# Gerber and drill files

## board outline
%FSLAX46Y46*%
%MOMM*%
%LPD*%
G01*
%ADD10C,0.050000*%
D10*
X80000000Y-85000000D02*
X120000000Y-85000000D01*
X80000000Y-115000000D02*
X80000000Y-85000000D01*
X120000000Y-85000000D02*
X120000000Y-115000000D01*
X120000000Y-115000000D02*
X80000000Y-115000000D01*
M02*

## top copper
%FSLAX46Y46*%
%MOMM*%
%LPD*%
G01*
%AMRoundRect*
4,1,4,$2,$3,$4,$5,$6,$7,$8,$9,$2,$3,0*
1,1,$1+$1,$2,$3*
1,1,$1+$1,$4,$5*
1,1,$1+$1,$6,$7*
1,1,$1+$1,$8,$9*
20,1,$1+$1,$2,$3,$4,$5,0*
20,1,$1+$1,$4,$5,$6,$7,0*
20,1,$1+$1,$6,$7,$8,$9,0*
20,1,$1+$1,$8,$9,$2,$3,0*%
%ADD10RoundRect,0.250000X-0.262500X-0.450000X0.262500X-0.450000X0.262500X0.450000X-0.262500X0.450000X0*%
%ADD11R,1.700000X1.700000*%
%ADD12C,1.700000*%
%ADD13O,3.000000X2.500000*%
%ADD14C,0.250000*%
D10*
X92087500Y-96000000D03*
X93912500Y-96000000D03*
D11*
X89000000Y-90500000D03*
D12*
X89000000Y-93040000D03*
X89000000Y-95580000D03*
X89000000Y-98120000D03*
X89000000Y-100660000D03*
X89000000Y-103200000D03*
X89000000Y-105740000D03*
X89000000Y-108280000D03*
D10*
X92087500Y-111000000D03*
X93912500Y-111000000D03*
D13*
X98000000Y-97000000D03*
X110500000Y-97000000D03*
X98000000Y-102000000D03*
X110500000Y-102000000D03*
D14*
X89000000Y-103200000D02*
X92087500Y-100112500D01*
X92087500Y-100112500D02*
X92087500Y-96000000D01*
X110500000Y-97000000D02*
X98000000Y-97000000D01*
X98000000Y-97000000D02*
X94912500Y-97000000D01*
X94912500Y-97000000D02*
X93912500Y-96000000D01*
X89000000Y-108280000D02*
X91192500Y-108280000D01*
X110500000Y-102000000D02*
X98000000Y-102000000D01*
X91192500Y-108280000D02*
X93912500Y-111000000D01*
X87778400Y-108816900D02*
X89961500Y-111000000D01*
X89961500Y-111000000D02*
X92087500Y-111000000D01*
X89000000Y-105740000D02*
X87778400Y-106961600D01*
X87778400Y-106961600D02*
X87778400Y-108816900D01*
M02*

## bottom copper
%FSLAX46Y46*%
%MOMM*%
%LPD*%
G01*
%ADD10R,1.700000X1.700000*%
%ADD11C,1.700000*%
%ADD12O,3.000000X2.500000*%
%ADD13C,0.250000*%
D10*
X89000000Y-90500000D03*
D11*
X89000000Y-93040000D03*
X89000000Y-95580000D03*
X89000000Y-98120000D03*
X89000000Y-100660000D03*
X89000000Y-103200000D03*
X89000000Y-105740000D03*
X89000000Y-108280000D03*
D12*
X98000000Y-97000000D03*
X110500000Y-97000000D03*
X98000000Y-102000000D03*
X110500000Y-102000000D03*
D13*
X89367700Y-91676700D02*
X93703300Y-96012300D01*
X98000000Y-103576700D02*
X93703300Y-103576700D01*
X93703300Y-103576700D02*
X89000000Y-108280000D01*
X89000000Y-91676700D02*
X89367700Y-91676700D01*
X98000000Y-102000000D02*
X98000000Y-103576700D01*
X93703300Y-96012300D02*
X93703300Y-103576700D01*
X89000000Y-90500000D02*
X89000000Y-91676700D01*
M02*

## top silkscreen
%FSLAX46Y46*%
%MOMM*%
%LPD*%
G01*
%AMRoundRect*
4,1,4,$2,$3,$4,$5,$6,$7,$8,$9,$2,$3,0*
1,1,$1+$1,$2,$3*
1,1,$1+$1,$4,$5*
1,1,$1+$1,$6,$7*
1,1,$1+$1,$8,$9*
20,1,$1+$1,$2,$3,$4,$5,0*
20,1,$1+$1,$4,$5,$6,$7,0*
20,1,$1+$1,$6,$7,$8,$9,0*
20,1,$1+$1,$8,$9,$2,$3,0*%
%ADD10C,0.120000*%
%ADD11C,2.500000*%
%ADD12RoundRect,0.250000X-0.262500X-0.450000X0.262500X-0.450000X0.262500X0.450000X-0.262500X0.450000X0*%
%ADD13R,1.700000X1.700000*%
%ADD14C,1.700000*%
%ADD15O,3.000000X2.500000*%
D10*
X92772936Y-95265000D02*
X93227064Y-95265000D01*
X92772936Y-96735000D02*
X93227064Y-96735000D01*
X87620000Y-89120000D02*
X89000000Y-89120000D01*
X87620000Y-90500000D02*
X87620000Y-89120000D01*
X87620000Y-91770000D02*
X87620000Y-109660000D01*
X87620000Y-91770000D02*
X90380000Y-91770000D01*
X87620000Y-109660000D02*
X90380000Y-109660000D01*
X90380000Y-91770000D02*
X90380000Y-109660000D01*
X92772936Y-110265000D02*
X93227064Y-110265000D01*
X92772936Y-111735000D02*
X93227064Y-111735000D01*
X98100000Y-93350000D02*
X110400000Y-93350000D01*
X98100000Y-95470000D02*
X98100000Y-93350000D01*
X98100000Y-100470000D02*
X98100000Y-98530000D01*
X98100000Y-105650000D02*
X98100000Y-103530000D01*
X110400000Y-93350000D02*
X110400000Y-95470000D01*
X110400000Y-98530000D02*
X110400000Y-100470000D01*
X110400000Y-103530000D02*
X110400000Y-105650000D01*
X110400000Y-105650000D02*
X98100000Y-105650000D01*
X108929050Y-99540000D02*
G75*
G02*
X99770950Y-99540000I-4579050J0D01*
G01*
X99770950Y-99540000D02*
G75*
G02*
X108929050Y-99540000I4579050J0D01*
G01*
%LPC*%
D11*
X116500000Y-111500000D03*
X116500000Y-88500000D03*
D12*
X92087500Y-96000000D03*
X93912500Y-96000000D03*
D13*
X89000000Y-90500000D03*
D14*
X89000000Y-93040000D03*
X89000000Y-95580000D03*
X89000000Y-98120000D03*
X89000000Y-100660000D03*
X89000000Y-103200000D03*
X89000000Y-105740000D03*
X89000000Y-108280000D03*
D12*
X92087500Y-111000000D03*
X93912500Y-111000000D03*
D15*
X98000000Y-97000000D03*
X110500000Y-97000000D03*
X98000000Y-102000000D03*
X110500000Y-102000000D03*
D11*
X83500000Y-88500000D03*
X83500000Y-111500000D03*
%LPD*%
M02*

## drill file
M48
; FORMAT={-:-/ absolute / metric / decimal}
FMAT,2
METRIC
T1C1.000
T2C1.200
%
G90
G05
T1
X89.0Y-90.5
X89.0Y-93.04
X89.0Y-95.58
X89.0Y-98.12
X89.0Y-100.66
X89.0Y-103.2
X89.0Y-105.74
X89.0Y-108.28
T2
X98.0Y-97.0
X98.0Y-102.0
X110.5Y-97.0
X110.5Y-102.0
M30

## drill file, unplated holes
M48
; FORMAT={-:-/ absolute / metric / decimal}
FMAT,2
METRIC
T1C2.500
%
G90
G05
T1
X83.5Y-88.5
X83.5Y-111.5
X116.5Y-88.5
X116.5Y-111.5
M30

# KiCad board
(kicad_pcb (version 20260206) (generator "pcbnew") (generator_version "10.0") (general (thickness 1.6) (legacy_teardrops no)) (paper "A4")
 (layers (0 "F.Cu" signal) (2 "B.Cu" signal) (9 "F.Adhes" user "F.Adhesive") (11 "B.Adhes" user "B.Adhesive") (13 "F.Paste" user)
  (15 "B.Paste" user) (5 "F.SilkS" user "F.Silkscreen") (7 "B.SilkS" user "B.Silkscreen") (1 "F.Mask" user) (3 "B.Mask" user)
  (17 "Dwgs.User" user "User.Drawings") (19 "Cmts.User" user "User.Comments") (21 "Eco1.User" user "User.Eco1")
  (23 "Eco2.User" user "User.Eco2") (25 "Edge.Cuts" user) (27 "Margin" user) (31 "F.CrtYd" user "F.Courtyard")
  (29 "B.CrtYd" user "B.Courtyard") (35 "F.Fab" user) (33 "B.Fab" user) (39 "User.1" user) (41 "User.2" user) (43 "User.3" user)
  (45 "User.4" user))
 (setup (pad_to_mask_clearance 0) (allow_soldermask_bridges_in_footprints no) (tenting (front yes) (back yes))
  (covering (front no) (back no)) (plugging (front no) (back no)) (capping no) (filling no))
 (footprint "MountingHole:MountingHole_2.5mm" (layer "F.Cu") (at 116.5 111.5)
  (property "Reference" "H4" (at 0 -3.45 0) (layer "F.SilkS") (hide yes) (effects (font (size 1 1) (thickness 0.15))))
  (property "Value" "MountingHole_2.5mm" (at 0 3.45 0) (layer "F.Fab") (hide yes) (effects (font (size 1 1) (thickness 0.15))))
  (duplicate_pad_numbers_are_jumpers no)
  (pad "" np_thru_hole circle (at 0 0) (size 2.5 2.5) (drill 2.5) (layers "*.Cu" "*.Mask")))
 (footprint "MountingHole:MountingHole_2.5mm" (layer "F.Cu") (at 116.5 88.5)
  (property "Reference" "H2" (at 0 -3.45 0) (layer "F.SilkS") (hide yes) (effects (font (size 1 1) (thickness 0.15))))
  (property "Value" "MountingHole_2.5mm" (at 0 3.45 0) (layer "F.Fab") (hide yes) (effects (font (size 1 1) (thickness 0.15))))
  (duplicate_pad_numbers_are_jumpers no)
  (pad "" np_thru_hole circle (at 0 0) (size 2.5 2.5) (drill 2.5) (layers "*.Cu" "*.Mask")))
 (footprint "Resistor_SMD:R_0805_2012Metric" (layer "F.Cu") (at 93 96)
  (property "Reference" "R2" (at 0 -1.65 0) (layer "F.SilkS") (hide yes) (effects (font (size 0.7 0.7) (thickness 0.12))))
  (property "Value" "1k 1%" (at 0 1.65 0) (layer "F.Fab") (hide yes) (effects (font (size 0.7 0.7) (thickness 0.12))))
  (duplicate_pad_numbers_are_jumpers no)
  (fp_line (start -0.227064 -0.735) (end 0.227064 -0.735) (stroke (width 0.12) (type solid)) (layer "F.SilkS"))
  (fp_line (start -0.227064 0.735) (end 0.227064 0.735) (stroke (width 0.12) (type solid)) (layer "F.SilkS"))
  (pad "1" smd roundrect (at -0.9125 0) (size 1.025 1.4) (layers "F.Cu" "F.Mask" "F.Paste") (roundrect_rratio 0.243902) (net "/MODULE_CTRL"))
  (pad "2" smd roundrect (at 0.9125 0) (size 1.025 1.4) (layers "F.Cu" "F.Mask" "F.Paste") (roundrect_rratio 0.243902) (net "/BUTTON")))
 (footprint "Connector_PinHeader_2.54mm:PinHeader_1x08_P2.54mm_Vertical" (layer "F.Cu") (at 89 90.5)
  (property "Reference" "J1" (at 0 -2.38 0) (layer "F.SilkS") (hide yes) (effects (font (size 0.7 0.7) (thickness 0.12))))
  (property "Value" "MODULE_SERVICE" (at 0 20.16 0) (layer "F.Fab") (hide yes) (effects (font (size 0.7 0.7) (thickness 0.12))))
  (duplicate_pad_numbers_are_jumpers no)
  (fp_line (start -1.38 -1.38) (end 0 -1.38) (stroke (width 0.12) (type solid)) (layer "F.SilkS"))
  (fp_line (start -1.38 0) (end -1.38 -1.38) (stroke (width 0.12) (type solid)) (layer "F.SilkS"))
  (fp_line (start -1.38 1.27) (end -1.38 19.16) (stroke (width 0.12) (type solid)) (layer "F.SilkS"))
  (fp_line (start -1.38 1.27) (end 1.38 1.27) (stroke (width 0.12) (type solid)) (layer "F.SilkS"))
  (fp_line (start -1.38 19.16) (end 1.38 19.16) (stroke (width 0.12) (type solid)) (layer "F.SilkS"))
  (fp_line (start 1.38 1.27) (end 1.38 19.16) (stroke (width 0.12) (type solid)) (layer "F.SilkS"))
  (pad "1" thru_hole rect (at 0 0) (size 1.7 1.7) (drill 1) (layers "*.Cu" "*.Mask") (remove_unused_layers no) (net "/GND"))
  (pad "2" thru_hole circle (at 0 2.54) (size 1.7 1.7) (drill 1) (layers "*.Cu" "*.Mask") (remove_unused_layers no)
   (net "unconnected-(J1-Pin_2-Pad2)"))
  (pad "3" thru_hole circle (at 0 5.08) (size 1.7 1.7) (drill 1) (layers "*.Cu" "*.Mask") (remove_unused_layers no)
   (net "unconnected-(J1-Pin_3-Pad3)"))
  (pad "4" thru_hole circle (at 0 7.62) (size 1.7 1.7) (drill 1) (layers "*.Cu" "*.Mask") (remove_unused_layers no)
   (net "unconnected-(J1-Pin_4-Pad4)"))
  (pad "5" thru_hole circle (at 0 10.16) (size 1.7 1.7) (drill 1) (layers "*.Cu" "*.Mask") (remove_unused_layers no)
   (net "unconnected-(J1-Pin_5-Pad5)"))
  (pad "6" thru_hole circle (at 0 12.7) (size 1.7 1.7) (drill 1) (layers "*.Cu" "*.Mask") (remove_unused_layers no) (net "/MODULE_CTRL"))
  (pad "7" thru_hole circle (at 0 15.24) (size 1.7 1.7) (drill 1) (layers "*.Cu" "*.Mask") (remove_unused_layers no) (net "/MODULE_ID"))
  (pad "8" thru_hole circle (at 0 17.78) (size 1.7 1.7) (drill 1) (layers "*.Cu" "*.Mask") (remove_unused_layers no) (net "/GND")))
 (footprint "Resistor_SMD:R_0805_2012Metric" (layer "F.Cu") (at 93 111)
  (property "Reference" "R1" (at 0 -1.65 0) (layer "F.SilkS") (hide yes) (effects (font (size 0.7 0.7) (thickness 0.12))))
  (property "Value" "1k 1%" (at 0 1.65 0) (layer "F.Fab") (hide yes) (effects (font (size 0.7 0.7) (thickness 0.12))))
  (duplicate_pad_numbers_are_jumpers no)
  (fp_line (start -0.227064 -0.735) (end 0.227064 -0.735) (stroke (width 0.12) (type solid)) (layer "F.SilkS"))
  (fp_line (start -0.227064 0.735) (end 0.227064 0.735) (stroke (width 0.12) (type solid)) (layer "F.SilkS"))
  (pad "1" smd roundrect (at -0.9125 0) (size 1.025 1.4) (layers "F.Cu" "F.Mask" "F.Paste") (roundrect_rratio 0.243902) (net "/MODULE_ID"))
  (pad "2" smd roundrect (at 0.9125 0) (size 1.025 1.4) (layers "F.Cu" "F.Mask" "F.Paste") (roundrect_rratio 0.243902) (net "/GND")))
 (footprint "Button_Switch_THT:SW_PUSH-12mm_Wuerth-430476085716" (layer "F.Cu") (at 98 97)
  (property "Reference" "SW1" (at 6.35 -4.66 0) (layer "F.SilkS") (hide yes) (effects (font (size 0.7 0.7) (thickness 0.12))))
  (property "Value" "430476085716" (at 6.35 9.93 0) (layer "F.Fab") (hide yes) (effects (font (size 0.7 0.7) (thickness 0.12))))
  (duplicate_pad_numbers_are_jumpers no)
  (fp_line (start 0.1 -3.65) (end 12.4 -3.65) (stroke (width 0.12) (type solid)) (layer "F.SilkS"))
  (fp_line (start 0.1 -1.53) (end 0.1 -3.65) (stroke (width 0.12) (type solid)) (layer "F.SilkS"))
  (fp_line (start 0.1 3.47) (end 0.1 1.53) (stroke (width 0.12) (type solid)) (layer "F.SilkS"))
  (fp_line (start 0.1 8.65) (end 0.1 6.53) (stroke (width 0.12) (type solid)) (layer "F.SilkS"))
  (fp_line (start 12.4 -3.65) (end 12.4 -1.53) (stroke (width 0.12) (type solid)) (layer "F.SilkS"))
  (fp_line (start 12.4 1.53) (end 12.4 3.47) (stroke (width 0.12) (type solid)) (layer "F.SilkS"))
  (fp_line (start 12.4 6.53) (end 12.4 8.65) (stroke (width 0.12) (type solid)) (layer "F.SilkS"))
  (fp_line (start 12.4 8.65) (end 0.1 8.65) (stroke (width 0.12) (type solid)) (layer "F.SilkS"))
  (fp_circle (center 6.35 2.54) (end 10.92905 2.54) (stroke (width 0.12) (type solid)) (fill no) (layer "F.SilkS"))
  (pad "1" thru_hole oval (at 0 0) (size 3 2.5) (drill 1.2) (layers "*.Cu" "*.Mask") (remove_unused_layers no) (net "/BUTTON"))
  (pad "1" thru_hole oval (at 12.5 0) (size 3 2.5) (drill 1.2) (layers "*.Cu" "*.Mask") (remove_unused_layers no) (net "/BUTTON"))
  (pad "2" thru_hole oval (at 0 5) (size 3 2.5) (drill 1.2) (layers "*.Cu" "*.Mask") (remove_unused_layers no) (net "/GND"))
  (pad "2" thru_hole oval (at 12.5 5) (size 3 2.5) (drill 1.2) (layers "*.Cu" "*.Mask") (remove_unused_layers no) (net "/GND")))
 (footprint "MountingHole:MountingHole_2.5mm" (layer "F.Cu") (at 83.5 88.5)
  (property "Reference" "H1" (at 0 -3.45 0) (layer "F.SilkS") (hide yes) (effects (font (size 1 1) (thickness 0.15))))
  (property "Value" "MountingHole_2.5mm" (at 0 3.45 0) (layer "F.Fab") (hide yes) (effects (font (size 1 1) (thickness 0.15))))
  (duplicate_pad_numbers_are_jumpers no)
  (pad "" np_thru_hole circle (at 0 0) (size 2.5 2.5) (drill 2.5) (layers "*.Cu" "*.Mask")))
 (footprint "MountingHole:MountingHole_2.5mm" (layer "F.Cu") (at 83.5 111.5)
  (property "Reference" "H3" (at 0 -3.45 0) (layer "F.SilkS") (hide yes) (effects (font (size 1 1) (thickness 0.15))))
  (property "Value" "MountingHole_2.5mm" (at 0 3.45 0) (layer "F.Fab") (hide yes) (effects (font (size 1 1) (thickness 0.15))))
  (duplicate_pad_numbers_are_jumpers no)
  (pad "" np_thru_hole circle (at 0 0) (size 2.5 2.5) (drill 2.5) (layers "*.Cu" "*.Mask")))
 (gr_line (start 80 85) (end 120 85) (stroke (width 0.05) (type default)) (layer "Edge.Cuts"))
 (gr_line (start 80 115) (end 80 85) (stroke (width 0.05) (type default)) (layer "Edge.Cuts"))
 (gr_line (start 120 85) (end 120 115) (stroke (width 0.05) (type default)) (layer "Edge.Cuts"))
 (gr_line (start 120 115) (end 80 115) (stroke (width 0.05) (type default)) (layer "Edge.Cuts"))
 (segment (start 89 103.2) (end 92.0875 100.1125) (width 0.25) (layer "F.Cu") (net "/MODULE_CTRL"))
 (segment (start 92.0875 100.1125) (end 92.0875 96) (width 0.25) (layer "F.Cu") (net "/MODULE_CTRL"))
 (segment (start 110.5 97) (end 98 97) (width 0.25) (layer "F.Cu") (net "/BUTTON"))
 (segment (start 98 97) (end 94.9125 97) (width 0.25) (layer "F.Cu") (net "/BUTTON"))
 (segment (start 94.9125 97) (end 93.9125 96) (width 0.25) (layer "F.Cu") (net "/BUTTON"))
 (segment (start 89 108.28) (end 91.1925 108.28) (width 0.25) (layer "F.Cu") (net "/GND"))
 (segment (start 110.5 102) (end 98 102) (width 0.25) (layer "F.Cu") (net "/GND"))
 (segment (start 91.1925 108.28) (end 93.9125 111) (width 0.25) (layer "F.Cu") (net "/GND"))
 (segment (start 89.3677 91.6767) (end 93.7033 96.0123) (width 0.25) (layer "B.Cu") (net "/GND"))
 (segment (start 98 103.5767) (end 93.7033 103.5767) (width 0.25) (layer "B.Cu") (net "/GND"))
 (segment (start 93.7033 103.5767) (end 89 108.28) (width 0.25) (layer "B.Cu") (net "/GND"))
 (segment (start 89 91.6767) (end 89.3677 91.6767) (width 0.25) (layer "B.Cu") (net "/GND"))
 (segment (start 98 102) (end 98 103.5767) (width 0.25) (layer "B.Cu") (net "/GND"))
 (segment (start 93.7033 96.0123) (end 93.7033 103.5767) (width 0.25) (layer "B.Cu") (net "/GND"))
 (segment (start 89 90.5) (end 89 91.6767) (width 0.25) (layer "B.Cu") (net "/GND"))
 (segment (start 87.7784 108.8169) (end 89.9615 111) (width 0.25) (layer "F.Cu") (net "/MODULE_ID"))
 (segment (start 89.9615 111) (end 92.0875 111) (width 0.25) (layer "F.Cu") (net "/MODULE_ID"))
 (segment (start 89 105.74) (end 87.7784 106.9616) (width 0.25) (layer "F.Cu") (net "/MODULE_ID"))
 (segment (start 87.7784 106.9616) (end 87.7784 108.8169) (width 0.25) (layer "F.Cu") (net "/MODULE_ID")))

